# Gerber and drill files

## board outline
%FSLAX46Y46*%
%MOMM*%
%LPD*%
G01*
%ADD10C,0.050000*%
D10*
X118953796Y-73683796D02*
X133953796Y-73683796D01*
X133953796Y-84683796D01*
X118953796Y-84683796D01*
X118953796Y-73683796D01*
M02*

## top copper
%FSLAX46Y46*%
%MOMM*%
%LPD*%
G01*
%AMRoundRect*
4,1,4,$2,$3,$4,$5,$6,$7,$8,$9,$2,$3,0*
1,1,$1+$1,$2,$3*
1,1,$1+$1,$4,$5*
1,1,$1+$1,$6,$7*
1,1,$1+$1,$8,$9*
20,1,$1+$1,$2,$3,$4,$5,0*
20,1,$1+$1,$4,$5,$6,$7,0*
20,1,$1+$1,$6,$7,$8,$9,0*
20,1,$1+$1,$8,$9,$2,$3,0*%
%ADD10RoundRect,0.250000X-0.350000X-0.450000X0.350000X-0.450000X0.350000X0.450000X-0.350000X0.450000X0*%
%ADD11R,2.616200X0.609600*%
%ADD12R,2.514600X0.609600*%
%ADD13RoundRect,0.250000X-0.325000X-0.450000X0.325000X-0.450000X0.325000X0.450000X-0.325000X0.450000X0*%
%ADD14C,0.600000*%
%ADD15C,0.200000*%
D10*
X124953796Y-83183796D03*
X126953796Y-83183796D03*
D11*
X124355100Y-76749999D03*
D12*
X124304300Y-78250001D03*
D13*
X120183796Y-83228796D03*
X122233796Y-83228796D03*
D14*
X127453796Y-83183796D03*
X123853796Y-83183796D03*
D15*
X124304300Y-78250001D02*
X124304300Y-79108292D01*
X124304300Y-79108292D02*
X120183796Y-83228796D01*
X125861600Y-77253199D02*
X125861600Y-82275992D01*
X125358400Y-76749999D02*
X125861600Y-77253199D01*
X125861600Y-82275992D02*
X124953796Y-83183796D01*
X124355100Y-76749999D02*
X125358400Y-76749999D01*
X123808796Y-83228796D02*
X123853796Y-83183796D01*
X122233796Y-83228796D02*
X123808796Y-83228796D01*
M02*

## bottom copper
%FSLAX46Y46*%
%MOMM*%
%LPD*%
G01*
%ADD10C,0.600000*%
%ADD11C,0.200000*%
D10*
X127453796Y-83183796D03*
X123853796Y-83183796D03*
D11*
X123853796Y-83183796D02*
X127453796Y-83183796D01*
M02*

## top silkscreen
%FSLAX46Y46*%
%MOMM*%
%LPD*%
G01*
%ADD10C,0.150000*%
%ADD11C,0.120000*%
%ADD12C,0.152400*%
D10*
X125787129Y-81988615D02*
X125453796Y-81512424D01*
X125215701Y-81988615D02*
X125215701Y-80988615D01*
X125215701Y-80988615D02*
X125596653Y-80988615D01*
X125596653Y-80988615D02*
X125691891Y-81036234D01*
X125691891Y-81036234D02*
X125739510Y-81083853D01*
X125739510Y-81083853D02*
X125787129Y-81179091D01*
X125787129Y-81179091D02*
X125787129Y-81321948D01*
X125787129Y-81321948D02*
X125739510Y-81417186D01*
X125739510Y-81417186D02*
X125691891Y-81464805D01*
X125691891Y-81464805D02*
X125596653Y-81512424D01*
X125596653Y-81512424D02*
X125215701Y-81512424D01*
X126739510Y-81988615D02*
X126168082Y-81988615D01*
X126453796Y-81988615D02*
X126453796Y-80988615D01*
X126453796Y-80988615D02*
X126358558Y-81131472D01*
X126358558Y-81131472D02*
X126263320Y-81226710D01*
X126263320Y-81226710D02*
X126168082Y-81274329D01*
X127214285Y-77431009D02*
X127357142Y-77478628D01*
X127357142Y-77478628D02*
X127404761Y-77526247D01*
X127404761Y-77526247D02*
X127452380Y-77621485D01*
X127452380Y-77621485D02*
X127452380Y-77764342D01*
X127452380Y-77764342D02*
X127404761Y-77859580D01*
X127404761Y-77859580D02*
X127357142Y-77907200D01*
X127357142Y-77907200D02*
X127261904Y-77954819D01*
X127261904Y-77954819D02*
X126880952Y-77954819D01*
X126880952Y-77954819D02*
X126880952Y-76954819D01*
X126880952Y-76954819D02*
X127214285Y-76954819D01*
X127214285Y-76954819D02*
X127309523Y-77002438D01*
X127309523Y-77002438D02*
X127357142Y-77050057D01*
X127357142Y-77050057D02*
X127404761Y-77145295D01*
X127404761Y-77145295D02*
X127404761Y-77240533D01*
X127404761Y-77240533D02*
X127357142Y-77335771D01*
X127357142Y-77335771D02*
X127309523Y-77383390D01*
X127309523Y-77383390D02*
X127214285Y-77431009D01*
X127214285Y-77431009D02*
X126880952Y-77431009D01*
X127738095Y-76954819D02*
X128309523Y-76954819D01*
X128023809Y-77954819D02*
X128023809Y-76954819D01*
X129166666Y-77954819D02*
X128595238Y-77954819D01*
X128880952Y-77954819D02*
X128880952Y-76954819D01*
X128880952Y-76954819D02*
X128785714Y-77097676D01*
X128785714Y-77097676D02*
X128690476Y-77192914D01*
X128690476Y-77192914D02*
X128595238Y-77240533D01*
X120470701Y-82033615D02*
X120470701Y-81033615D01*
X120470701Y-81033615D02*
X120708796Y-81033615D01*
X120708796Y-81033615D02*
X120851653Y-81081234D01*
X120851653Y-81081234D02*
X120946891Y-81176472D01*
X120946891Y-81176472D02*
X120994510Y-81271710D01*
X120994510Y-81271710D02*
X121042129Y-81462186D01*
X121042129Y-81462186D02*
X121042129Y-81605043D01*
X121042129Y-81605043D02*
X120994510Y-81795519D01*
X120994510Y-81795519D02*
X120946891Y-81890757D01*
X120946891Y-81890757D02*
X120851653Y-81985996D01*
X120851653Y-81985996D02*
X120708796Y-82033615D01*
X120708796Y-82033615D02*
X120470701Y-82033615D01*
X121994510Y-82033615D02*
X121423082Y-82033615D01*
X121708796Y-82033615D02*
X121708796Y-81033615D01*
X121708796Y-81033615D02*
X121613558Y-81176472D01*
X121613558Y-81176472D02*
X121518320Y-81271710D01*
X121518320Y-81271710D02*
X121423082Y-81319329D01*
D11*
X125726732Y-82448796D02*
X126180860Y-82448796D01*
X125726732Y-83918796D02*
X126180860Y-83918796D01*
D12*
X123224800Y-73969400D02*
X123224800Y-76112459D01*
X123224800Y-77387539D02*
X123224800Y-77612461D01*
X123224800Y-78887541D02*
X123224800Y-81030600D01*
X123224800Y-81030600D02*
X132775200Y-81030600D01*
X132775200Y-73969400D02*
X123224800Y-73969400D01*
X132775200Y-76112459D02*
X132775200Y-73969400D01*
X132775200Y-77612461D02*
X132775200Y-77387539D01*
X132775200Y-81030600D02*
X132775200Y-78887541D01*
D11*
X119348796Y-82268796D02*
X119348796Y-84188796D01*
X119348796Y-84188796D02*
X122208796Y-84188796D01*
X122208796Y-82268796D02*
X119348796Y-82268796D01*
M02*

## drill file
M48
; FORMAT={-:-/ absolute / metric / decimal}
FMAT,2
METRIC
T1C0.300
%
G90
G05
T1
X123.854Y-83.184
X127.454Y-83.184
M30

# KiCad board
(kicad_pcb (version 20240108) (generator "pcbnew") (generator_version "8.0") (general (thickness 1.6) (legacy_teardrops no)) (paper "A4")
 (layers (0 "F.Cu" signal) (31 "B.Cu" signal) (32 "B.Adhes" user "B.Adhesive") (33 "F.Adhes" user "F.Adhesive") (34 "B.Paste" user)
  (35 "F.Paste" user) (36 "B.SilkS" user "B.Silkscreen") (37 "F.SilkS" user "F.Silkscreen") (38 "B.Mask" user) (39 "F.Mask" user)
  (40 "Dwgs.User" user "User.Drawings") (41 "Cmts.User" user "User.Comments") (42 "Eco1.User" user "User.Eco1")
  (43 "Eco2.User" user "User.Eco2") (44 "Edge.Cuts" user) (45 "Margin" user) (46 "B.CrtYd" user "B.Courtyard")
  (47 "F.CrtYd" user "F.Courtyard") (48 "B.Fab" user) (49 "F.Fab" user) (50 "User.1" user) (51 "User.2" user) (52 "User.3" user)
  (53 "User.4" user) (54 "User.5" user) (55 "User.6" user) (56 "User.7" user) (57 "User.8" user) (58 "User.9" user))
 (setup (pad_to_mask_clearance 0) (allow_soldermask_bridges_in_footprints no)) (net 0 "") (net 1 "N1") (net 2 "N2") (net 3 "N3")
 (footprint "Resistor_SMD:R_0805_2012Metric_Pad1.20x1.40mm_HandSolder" (layer "F.Cu") (at 125.953796 83.183796)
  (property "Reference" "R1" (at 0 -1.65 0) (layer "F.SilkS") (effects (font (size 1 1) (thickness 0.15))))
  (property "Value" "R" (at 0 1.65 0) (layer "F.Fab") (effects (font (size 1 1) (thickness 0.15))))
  (fp_line (start -0.227064 -0.735) (end 0.227064 -0.735) (stroke (width 0.12) (type solid)) (layer "F.SilkS"))
  (fp_line (start -0.227064 0.735) (end 0.227064 0.735) (stroke (width 0.12) (type solid)) (layer "F.SilkS"))
  (pad "1" smd roundrect (at -1 0) (size 1.2 1.4) (layers "F.Cu" "F.Paste" "F.Mask") (roundrect_rratio 0.208333) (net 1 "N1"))
  (pad "2" smd roundrect (at 1 0) (size 1.2 1.4) (layers "F.Cu" "F.Paste" "F.Mask") (roundrect_rratio 0.208333) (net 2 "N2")))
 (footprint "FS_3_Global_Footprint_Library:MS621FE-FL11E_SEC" (layer "F.Cu") (at 128 77.5)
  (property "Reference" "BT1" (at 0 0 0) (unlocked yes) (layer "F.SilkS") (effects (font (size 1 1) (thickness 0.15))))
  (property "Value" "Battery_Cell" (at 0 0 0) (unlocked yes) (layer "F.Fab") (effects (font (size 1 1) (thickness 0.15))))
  (fp_line (start -4.7752 -3.5306) (end -4.7752 -1.387541) (stroke (width 0.1524) (type solid)) (layer "F.SilkS"))
  (fp_line (start -4.7752 -0.112461) (end -4.7752 0.112461) (stroke (width 0.1524) (type solid)) (layer "F.SilkS"))
  (fp_line (start -4.7752 1.387541) (end -4.7752 3.5306) (stroke (width 0.1524) (type solid)) (layer "F.SilkS"))
  (fp_line (start -4.7752 3.5306) (end 4.7752 3.5306) (stroke (width 0.1524) (type solid)) (layer "F.SilkS"))
  (fp_line (start 4.7752 -3.5306) (end -4.7752 -3.5306) (stroke (width 0.1524) (type solid)) (layer "F.SilkS"))
  (fp_line (start 4.7752 -1.387541) (end 4.7752 -3.5306) (stroke (width 0.1524) (type solid)) (layer "F.SilkS"))
  (fp_line (start 4.7752 0.112461) (end 4.7752 -0.112461) (stroke (width 0.1524) (type solid)) (layer "F.SilkS"))
  (fp_line (start 4.7752 3.5306) (end 4.7752 1.387541) (stroke (width 0.1524) (type solid)) (layer "F.SilkS"))
  (pad "1" smd rect (at -3.6449 -0.750001) (size 2.6162 0.6096) (layers "F.Cu" "F.Paste" "F.Mask") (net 1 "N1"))
  (pad "2" smd rect (at -3.6957 0.750001) (size 2.5146 0.6096) (layers "F.Cu" "F.Paste" "F.Mask") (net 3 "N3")))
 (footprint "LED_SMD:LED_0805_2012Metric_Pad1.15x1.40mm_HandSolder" (layer "F.Cu") (at 121.208796 83.228796)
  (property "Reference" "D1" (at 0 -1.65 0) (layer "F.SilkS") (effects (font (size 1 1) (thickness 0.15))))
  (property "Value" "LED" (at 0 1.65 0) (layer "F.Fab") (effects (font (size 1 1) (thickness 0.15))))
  (fp_line (start -1.86 -0.96) (end -1.86 0.96) (stroke (width 0.12) (type solid)) (layer "F.SilkS"))
  (fp_line (start -1.86 0.96) (end 1 0.96) (stroke (width 0.12) (type solid)) (layer "F.SilkS"))
  (fp_line (start 1 -0.96) (end -1.86 -0.96) (stroke (width 0.12) (type solid)) (layer "F.SilkS"))
  (pad "1" smd roundrect (at -1.025 0) (size 1.15 1.4) (layers "F.Cu" "F.Paste" "F.Mask") (roundrect_rratio 0.217391) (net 3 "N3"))
  (pad "2" smd roundrect (at 1.025 0) (size 1.15 1.4) (layers "F.Cu" "F.Paste" "F.Mask") (roundrect_rratio 0.217391) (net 2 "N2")))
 (gr_rect (start 118.953796 73.683796) (end 133.953796 84.683796) (stroke (width 0.05) (type default)) (fill none) (layer "Edge.Cuts"))
 (segment (start 124.3043 78.250001) (end 124.3043 79.108292) (width 0.2) (layer "F.Cu") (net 3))
 (segment (start 124.3043 79.108292) (end 120.183796 83.228796) (width 0.2) (layer "F.Cu") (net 3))
 (segment (start 125.8616 77.253199) (end 125.8616 82.275992) (width 0.2) (layer "F.Cu") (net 1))
 (segment (start 125.3584 76.749999) (end 125.8616 77.253199) (width 0.2) (layer "F.Cu") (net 1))
 (segment (start 125.8616 82.275992) (end 124.953796 83.183796) (width 0.2) (layer "F.Cu") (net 1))
 (segment (start 124.3551 76.749999) (end 125.3584 76.749999) (width 0.2) (layer "F.Cu") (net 1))
 (segment (start 123.808796 83.228796) (end 123.853796 83.183796) (width 0.2) (layer "F.Cu") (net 2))
 (segment (start 122.233796 83.228796) (end 123.808796 83.228796) (width 0.2) (layer "F.Cu") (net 2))
 (via (at 127.453796 83.183796) (size 0.6) (drill 0.3) (layers "F.Cu" "B.Cu") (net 2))
 (via (at 123.853796 83.183796) (size 0.6) (drill 0.3) (layers "F.Cu" "B.Cu") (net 2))
 (segment (start 123.853796 83.183796) (end 127.453796 83.183796) (width 0.2) (layer "B.Cu") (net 2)))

